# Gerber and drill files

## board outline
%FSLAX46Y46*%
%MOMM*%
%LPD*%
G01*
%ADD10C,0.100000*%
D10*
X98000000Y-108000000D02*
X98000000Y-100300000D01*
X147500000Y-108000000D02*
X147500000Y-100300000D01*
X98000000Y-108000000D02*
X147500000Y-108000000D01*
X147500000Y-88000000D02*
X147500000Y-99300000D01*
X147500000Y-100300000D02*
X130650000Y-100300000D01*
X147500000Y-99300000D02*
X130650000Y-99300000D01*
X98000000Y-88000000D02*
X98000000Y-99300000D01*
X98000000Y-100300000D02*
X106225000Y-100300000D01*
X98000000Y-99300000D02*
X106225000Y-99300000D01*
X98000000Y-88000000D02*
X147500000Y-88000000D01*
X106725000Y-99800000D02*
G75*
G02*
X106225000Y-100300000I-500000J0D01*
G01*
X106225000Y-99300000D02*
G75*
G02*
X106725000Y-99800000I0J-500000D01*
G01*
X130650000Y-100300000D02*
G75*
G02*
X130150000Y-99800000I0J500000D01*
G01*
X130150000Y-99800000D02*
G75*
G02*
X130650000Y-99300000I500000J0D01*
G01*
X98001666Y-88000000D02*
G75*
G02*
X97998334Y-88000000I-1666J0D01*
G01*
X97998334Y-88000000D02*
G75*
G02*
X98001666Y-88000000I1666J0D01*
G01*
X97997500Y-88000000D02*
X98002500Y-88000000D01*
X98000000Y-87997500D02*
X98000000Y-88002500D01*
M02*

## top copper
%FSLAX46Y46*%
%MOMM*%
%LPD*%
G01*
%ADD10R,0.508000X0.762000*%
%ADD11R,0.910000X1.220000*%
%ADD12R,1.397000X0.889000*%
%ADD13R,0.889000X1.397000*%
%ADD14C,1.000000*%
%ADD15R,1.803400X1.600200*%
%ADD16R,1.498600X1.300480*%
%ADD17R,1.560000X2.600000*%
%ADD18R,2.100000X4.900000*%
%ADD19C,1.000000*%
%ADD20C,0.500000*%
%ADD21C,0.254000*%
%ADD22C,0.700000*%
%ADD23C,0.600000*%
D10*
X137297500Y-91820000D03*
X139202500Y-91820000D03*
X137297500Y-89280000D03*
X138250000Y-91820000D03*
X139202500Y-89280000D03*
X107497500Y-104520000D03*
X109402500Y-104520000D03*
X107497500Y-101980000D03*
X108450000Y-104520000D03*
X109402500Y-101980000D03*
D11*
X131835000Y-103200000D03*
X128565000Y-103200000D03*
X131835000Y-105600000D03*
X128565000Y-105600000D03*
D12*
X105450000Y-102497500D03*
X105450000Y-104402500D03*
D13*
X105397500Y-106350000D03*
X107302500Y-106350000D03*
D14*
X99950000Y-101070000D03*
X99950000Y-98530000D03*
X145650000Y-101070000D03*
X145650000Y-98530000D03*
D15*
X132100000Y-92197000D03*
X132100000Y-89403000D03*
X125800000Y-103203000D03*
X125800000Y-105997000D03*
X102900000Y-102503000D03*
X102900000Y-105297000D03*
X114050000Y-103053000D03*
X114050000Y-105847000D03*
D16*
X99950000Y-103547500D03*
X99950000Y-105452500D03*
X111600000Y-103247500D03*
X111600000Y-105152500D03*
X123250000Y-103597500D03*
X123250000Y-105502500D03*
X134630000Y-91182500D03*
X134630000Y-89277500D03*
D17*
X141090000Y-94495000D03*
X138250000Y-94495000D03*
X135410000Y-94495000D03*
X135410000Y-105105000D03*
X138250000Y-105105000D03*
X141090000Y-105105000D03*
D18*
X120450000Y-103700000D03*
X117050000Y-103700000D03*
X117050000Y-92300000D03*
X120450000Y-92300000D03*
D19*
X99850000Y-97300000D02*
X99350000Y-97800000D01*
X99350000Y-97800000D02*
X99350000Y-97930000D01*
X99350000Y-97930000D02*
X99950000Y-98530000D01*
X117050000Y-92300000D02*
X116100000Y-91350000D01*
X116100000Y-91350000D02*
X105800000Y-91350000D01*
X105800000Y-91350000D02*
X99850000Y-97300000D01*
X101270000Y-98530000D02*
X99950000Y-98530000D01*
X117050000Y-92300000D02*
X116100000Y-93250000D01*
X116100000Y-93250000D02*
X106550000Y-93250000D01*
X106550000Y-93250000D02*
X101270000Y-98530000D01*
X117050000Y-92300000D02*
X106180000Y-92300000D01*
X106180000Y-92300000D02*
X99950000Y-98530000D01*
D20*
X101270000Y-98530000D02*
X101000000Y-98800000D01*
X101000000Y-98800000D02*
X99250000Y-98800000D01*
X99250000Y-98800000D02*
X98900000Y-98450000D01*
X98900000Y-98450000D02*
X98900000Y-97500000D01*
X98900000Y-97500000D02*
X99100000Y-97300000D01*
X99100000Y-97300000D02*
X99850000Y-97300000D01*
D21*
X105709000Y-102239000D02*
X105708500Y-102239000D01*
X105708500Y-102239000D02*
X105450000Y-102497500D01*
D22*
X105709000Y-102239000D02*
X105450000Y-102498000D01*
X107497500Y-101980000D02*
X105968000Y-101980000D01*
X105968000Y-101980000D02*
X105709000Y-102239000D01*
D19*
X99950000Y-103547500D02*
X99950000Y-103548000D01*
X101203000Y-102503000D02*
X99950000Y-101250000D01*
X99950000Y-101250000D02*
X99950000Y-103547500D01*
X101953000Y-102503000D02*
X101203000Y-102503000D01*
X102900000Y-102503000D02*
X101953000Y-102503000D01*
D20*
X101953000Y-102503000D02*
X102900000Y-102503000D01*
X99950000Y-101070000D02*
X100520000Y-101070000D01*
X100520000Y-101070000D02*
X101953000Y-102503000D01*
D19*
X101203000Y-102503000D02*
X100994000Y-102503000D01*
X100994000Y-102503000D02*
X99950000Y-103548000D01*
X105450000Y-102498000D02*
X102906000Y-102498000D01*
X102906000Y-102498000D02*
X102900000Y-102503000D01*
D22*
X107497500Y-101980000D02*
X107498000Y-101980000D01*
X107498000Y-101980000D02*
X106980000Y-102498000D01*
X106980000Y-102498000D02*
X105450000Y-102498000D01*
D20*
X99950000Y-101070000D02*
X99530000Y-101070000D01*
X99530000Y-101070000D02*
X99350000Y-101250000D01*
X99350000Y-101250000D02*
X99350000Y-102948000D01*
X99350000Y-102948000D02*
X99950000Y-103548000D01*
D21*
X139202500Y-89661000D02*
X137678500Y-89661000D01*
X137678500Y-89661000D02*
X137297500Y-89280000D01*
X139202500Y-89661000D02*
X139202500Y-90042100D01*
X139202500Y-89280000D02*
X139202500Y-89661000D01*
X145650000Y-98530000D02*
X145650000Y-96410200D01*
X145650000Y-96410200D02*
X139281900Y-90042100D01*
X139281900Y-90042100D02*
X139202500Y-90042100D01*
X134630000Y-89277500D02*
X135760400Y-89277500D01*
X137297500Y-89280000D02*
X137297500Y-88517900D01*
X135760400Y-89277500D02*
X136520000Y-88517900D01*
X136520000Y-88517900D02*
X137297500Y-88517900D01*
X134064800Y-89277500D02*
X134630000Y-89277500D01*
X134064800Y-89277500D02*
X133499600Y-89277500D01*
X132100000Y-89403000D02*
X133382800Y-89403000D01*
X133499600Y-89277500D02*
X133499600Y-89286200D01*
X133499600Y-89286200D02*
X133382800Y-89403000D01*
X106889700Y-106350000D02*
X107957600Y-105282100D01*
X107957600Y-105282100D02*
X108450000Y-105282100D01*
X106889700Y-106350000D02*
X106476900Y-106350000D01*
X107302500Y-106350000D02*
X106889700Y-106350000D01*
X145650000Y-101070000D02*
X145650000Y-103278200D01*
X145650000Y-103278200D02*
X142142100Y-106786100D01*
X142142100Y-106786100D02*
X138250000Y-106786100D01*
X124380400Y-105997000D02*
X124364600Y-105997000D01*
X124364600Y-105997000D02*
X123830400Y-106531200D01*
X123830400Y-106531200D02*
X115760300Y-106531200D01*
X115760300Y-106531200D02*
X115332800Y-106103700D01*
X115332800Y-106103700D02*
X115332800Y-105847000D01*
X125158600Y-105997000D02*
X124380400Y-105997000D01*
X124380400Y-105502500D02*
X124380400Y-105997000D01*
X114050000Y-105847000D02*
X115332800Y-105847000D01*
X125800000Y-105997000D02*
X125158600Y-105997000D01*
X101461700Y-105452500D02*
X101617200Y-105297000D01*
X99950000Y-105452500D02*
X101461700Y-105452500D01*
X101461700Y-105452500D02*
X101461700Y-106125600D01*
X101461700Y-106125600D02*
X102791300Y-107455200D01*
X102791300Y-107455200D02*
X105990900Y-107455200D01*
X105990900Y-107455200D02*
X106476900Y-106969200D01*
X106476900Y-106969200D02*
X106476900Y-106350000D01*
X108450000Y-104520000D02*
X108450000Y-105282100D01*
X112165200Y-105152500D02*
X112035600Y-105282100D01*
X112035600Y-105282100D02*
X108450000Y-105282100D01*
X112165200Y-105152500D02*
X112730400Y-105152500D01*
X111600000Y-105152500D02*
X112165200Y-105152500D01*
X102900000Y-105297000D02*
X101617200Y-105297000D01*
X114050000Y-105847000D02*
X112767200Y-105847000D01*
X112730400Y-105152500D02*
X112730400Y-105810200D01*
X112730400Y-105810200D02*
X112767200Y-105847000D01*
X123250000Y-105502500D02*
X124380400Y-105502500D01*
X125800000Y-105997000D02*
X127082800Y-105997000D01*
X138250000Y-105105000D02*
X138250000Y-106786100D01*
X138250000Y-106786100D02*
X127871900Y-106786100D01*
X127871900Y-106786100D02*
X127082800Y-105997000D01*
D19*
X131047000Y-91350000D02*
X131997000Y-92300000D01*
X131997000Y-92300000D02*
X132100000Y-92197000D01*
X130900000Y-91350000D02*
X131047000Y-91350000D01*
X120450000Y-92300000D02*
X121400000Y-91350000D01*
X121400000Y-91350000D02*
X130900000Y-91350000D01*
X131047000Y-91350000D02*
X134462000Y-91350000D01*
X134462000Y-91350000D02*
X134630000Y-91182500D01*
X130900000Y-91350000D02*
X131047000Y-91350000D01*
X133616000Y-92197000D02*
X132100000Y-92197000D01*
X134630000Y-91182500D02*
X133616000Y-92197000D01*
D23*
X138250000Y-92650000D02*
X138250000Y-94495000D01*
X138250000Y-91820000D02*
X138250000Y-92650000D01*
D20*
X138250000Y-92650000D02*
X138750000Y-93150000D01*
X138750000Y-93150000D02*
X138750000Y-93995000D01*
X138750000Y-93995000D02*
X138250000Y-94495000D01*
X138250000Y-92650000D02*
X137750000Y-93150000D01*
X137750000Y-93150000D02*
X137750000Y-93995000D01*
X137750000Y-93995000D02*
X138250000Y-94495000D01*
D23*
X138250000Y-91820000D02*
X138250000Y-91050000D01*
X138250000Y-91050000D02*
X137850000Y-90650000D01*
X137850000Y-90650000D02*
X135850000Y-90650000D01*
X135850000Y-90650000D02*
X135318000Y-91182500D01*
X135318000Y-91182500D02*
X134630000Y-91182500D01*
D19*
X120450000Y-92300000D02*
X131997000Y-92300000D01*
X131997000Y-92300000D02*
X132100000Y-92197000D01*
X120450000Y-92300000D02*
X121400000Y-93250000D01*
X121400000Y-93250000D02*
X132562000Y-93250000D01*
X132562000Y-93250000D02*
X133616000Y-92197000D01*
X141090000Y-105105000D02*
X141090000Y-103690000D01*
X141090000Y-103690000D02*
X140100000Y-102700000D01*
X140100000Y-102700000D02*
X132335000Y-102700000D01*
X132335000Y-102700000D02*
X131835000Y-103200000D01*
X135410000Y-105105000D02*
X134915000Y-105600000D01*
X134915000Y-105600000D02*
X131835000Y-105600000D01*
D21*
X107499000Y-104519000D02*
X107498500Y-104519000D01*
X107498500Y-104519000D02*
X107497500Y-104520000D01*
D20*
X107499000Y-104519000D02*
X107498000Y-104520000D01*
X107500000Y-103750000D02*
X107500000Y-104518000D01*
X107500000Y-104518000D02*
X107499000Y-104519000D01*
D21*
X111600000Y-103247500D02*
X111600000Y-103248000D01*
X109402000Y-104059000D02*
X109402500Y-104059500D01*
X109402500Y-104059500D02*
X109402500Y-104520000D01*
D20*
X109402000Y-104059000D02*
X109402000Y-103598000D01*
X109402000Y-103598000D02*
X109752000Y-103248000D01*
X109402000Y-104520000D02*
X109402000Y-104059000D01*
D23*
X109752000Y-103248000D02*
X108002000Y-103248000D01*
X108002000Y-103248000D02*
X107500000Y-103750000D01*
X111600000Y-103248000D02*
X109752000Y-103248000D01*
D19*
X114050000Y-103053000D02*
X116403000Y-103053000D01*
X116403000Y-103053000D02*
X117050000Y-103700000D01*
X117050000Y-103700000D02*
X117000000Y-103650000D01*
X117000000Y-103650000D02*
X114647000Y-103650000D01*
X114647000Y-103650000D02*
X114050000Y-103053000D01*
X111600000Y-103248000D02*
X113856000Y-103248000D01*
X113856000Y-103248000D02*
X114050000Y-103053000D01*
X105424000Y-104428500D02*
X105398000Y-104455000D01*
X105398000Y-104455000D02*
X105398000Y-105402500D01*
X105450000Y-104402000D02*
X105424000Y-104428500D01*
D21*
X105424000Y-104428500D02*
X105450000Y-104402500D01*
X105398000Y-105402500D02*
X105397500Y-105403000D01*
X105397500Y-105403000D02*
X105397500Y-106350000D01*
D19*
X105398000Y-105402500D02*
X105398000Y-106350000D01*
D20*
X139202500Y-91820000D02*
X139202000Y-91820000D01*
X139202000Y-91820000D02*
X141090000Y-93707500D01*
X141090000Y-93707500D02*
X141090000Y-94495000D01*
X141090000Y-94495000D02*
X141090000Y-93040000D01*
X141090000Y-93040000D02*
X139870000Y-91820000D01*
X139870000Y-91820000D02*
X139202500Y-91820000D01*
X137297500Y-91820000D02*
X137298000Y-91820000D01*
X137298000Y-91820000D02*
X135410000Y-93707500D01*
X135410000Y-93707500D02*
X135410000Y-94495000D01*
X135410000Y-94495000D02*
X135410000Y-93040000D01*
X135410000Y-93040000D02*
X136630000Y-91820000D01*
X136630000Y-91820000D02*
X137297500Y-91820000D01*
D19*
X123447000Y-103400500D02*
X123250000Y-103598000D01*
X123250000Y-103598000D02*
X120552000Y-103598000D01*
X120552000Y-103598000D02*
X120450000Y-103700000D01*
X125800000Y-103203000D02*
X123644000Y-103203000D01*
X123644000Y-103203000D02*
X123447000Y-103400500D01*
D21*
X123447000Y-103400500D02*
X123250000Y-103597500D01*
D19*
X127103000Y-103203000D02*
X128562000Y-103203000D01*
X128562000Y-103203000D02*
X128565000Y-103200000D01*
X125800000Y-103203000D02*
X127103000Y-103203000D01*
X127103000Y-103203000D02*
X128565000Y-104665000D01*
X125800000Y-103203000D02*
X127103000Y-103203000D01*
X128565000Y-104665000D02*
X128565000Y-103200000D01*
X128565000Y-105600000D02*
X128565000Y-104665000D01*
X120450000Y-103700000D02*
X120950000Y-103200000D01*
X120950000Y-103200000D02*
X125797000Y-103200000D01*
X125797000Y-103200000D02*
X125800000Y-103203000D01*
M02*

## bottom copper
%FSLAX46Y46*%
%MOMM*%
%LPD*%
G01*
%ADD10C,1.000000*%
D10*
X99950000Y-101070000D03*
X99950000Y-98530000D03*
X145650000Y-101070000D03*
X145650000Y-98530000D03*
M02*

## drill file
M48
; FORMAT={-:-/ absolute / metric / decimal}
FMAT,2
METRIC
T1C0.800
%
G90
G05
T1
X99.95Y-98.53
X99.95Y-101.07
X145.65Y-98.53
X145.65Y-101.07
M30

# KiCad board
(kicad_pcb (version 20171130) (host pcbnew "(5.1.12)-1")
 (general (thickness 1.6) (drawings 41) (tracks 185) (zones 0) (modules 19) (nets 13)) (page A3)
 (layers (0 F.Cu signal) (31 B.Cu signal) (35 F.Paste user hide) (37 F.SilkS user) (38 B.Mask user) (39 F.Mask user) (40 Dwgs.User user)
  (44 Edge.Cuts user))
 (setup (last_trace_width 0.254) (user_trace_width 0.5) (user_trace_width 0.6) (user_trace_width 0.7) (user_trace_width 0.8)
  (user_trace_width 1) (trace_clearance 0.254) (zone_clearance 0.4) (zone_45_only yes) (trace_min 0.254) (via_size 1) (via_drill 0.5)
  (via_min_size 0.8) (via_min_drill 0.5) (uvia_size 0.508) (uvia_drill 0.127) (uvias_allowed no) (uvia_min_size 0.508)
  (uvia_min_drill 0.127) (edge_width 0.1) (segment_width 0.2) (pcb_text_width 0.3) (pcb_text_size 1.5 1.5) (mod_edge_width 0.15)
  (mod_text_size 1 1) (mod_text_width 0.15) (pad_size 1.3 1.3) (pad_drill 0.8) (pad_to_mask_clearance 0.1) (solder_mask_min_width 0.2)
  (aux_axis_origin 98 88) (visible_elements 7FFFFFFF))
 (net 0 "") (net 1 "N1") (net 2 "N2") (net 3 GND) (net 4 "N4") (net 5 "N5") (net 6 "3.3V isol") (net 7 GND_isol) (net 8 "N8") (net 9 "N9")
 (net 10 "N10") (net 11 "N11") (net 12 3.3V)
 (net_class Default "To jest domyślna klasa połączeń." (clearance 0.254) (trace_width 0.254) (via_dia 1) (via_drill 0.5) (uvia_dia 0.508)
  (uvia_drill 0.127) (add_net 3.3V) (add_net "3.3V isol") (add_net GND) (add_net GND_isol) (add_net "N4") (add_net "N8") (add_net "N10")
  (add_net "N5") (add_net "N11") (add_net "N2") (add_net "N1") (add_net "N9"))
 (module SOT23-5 (layer F.Cu) (at 138.25 90.55)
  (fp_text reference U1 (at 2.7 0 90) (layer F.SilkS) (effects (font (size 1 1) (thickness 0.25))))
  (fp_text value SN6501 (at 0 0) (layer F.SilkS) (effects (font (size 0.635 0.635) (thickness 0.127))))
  (pad 1 smd rect (at -0.9525 1.27) (size 0.508 0.762) (layers F.Cu F.Paste F.Mask) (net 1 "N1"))
  (pad 3 smd rect (at 0.9525 1.27) (size 0.508 0.762) (layers F.Cu F.Paste F.Mask) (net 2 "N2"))
  (pad 5 smd rect (at -0.9525 -1.27) (size 0.508 0.762) (layers F.Cu F.Paste F.Mask) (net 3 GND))
  (pad 2 smd rect (at 0 1.27) (size 0.508 0.762) (layers F.Cu F.Paste F.Mask) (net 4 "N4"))
  (pad 4 smd rect (at 0.9525 -1.27) (size 0.508 0.762) (layers F.Cu F.Paste F.Mask) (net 3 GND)))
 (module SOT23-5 (layer F.Cu) (at 108.45 103.25)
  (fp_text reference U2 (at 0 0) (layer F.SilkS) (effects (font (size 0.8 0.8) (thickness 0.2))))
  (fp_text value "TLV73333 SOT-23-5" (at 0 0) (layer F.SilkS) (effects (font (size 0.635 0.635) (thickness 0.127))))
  (pad 1 smd rect (at -0.9525 1.27) (size 0.508 0.762) (layers F.Cu F.Paste F.Mask) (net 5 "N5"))
  (pad 3 smd rect (at 0.9525 1.27) (size 0.508 0.762) (layers F.Cu F.Paste F.Mask) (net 5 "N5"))
  (pad 5 smd rect (at -0.9525 -1.27) (size 0.508 0.762) (layers F.Cu F.Paste F.Mask) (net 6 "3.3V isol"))
  (pad 2 smd rect (at 0 1.27) (size 0.508 0.762) (layers F.Cu F.Paste F.Mask) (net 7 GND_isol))
  (pad 4 smd rect (at 0.9525 -1.27) (size 0.508 0.762) (layers F.Cu F.Paste F.Mask)))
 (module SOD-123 (layer F.Cu) (at 130.2 103.2 180)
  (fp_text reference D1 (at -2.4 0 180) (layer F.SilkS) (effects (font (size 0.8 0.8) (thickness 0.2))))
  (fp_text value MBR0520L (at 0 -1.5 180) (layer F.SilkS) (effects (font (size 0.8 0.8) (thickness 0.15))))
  (pad 1 smd rect (at -1.635 0 180) (size 0.91 1.22) (layers F.Cu F.Paste F.Mask) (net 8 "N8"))
  (pad 2 smd rect (at 1.635 0 180) (size 0.91 1.22) (layers F.Cu F.Paste F.Mask) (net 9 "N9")))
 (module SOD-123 (layer F.Cu) (at 130.2 105.6 180)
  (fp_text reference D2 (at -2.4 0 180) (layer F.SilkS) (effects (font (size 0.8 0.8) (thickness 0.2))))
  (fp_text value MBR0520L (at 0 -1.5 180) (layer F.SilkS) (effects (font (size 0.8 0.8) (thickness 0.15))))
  (pad 1 smd rect (at -1.635 0 180) (size 0.91 1.22) (layers F.Cu F.Paste F.Mask) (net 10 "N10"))
  (pad 2 smd rect (at 1.635 0 180) (size 0.91 1.22) (layers F.Cu F.Paste F.Mask) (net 9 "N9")))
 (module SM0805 (layer F.Cu) (at 105.45 103.45 270)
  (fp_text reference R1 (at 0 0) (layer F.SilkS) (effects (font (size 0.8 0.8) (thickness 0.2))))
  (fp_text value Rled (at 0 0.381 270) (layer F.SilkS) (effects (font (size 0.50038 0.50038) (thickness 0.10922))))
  (pad 1 smd rect (at -0.9525 0 270) (size 0.889 1.397) (layers F.Cu F.Paste F.Mask) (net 6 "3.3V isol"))
  (pad 2 smd rect (at 0.9525 0 270) (size 0.889 1.397) (layers F.Cu F.Paste F.Mask) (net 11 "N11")))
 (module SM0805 (layer F.Cu) (at 106.35 106.35)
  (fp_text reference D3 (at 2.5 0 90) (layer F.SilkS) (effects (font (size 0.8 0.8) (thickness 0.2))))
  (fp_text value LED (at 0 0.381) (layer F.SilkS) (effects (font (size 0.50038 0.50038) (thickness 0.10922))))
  (pad 1 smd rect (at -0.9525 0) (size 0.889 1.397) (layers F.Cu F.Paste F.Mask) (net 11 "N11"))
  (pad 2 smd rect (at 0.9525 0) (size 0.889 1.397) (layers F.Cu F.Paste F.Mask) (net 7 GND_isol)))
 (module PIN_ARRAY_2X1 (layer F.Cu) (at 99.95 99.8 90)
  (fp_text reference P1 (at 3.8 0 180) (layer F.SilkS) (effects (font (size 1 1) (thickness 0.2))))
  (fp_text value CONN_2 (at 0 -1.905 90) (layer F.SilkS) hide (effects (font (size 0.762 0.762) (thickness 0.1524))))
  (pad 1 thru_hole circle (at -1.27 0 90) (size 1 1) (drill 0.8) (layers *.Cu *.Mask F.SilkS) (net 6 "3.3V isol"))
  (pad 2 thru_hole circle (at 1.27 0 90) (size 1 1) (drill 0.8) (layers *.Cu *.Mask F.SilkS) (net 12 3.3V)))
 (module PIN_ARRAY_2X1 (layer F.Cu) (at 145.65 99.8 90)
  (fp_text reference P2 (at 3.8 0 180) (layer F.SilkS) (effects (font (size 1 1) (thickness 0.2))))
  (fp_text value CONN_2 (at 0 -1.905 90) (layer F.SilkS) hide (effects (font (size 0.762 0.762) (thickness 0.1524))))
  (pad 1 thru_hole circle (at -1.27 0 90) (size 1 1) (drill 0.8) (layers *.Cu *.Mask F.SilkS) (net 7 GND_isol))
  (pad 2 thru_hole circle (at 1.27 0 90) (size 1 1) (drill 0.8) (layers *.Cu *.Mask F.SilkS) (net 3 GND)))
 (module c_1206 (layer F.Cu) (at 132.1 90.8 270)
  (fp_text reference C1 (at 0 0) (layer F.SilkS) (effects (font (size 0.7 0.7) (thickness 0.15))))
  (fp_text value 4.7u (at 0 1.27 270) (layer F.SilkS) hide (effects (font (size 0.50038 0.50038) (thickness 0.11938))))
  (pad 1 smd rect (at 1.397 0 270) (size 1.6002 1.8034) (layers F.Cu F.Paste F.Mask) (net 4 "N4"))
  (pad 2 smd rect (at -1.397 0 270) (size 1.6002 1.8034) (layers F.Cu F.Paste F.Mask) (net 3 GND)))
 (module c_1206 (layer F.Cu) (at 125.8 104.6 90)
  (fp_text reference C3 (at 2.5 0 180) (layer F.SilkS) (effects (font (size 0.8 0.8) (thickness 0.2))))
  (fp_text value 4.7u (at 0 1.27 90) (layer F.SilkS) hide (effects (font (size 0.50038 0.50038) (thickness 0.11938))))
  (pad 1 smd rect (at 1.397 0 90) (size 1.6002 1.8034) (layers F.Cu F.Paste F.Mask) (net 9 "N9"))
  (pad 2 smd rect (at -1.397 0 90) (size 1.6002 1.8034) (layers F.Cu F.Paste F.Mask) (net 7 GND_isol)))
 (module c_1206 (layer F.Cu) (at 102.9 103.9 90)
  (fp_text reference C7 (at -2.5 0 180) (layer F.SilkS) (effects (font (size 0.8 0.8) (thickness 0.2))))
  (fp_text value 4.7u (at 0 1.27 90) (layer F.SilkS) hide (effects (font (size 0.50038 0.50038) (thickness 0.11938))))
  (pad 1 smd rect (at 1.397 0 90) (size 1.6002 1.8034) (layers F.Cu F.Paste F.Mask) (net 6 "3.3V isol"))
  (pad 2 smd rect (at -1.397 0 90) (size 1.6002 1.8034) (layers F.Cu F.Paste F.Mask) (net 7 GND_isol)))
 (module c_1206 (layer F.Cu) (at 114.05 104.45 90)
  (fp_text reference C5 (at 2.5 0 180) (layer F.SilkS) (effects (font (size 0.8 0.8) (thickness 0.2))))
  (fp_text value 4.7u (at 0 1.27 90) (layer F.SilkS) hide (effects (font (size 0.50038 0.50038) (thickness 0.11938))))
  (pad 1 smd rect (at 1.397 0 90) (size 1.6002 1.8034) (layers F.Cu F.Paste F.Mask) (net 5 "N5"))
  (pad 2 smd rect (at -1.397 0 90) (size 1.6002 1.8034) (layers F.Cu F.Paste F.Mask) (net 7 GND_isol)))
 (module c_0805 (layer F.Cu) (at 99.95 104.5 90)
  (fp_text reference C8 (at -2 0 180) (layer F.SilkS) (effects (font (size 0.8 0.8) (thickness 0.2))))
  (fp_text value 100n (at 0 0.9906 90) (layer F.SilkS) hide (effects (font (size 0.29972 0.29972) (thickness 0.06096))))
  (pad 1 smd rect (at 0.9525 0 90) (size 1.30048 1.4986) (layers F.Cu F.Paste F.Mask) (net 6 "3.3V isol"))
  (pad 2 smd rect (at -0.9525 0 90) (size 1.30048 1.4986) (layers F.Cu F.Paste F.Mask) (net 7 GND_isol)))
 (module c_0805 (layer F.Cu) (at 111.6 104.2 90)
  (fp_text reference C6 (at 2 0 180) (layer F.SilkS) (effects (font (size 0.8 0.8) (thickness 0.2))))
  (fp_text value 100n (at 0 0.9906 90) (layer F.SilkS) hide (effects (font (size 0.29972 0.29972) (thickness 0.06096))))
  (pad 1 smd rect (at 0.9525 0 90) (size 1.30048 1.4986) (layers F.Cu F.Paste F.Mask) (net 5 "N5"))
  (pad 2 smd rect (at -0.9525 0 90) (size 1.30048 1.4986) (layers F.Cu F.Paste F.Mask) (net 7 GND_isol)))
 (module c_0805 (layer F.Cu) (at 123.25 104.55 90)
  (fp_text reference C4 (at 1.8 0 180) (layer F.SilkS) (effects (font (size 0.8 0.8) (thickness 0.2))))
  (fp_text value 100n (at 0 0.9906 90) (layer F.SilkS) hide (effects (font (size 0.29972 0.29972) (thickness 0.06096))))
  (pad 1 smd rect (at 0.9525 0 90) (size 1.30048 1.4986) (layers F.Cu F.Paste F.Mask) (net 9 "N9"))
  (pad 2 smd rect (at -0.9525 0 90) (size 1.30048 1.4986) (layers F.Cu F.Paste F.Mask) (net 7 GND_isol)))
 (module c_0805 (layer F.Cu) (at 134.63 90.23 270)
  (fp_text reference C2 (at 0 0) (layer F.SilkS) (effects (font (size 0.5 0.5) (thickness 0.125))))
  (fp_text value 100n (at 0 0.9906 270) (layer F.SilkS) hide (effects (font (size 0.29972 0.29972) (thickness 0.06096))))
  (pad 1 smd rect (at 0.9525 0 270) (size 1.30048 1.4986) (layers F.Cu F.Paste F.Mask) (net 4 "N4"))
  (pad 2 smd rect (at -0.9525 0 270) (size 1.30048 1.4986) (layers F.Cu F.Paste F.Mask) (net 3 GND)))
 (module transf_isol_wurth (layer F.Cu) (at 138.25 99.8 270)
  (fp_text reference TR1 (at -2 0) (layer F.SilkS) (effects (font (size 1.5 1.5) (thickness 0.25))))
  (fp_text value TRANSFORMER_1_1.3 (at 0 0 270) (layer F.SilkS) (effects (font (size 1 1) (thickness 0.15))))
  (pad 1 smd rect (at -5.305 -2.84 270) (size 2.6 1.56) (layers F.Cu F.Paste F.Mask) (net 2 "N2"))
  (pad 2 smd rect (at -5.305 0 270) (size 2.6 1.56) (layers F.Cu F.Paste F.Mask) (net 4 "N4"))
  (pad 3 smd rect (at -5.305 2.84 270) (size 2.6 1.56) (layers F.Cu F.Paste F.Mask) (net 1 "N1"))
  (pad 4 smd rect (at 5.305 2.84 270) (size 2.6 1.56) (layers F.Cu F.Paste F.Mask) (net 10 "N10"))
  (pad 5 smd rect (at 5.305 0 270) (size 2.6 1.56) (layers F.Cu F.Paste F.Mask) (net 7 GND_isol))
  (pad 6 smd rect (at 5.305 -2.84 270) (size 2.6 1.56) (layers F.Cu F.Paste F.Mask) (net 8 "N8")))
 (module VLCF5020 (layer F.Cu) (at 118.75 103.7 180)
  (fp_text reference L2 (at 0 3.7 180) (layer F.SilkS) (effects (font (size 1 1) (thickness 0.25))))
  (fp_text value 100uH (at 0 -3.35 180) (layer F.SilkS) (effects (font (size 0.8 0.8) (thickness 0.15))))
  (pad 1 smd rect (at -1.7 0 180) (size 2.1 4.9) (layers F.Cu F.Paste F.Mask) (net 9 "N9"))
  (pad 2 smd rect (at 1.7 0 180) (size 2.1 4.9) (layers F.Cu F.Paste F.Mask) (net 5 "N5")))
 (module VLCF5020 (layer F.Cu) (at 118.75 92.3)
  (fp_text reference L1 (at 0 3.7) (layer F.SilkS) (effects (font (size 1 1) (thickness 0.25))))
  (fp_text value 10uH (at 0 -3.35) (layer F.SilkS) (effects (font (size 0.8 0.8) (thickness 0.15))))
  (pad 1 smd rect (at -1.7 0) (size 2.1 4.9) (layers F.Cu F.Paste F.Mask) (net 12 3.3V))
  (pad 2 smd rect (at 1.7 0) (size 2.1 4.9) (layers F.Cu F.Paste F.Mask) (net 4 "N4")))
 (gr_line (start 98 108) (end 98 100.3) (angle 90) (layer Edge.Cuts) (width 0.1))
 (gr_line (start 147.5 108) (end 147.5 100.3) (angle 90) (layer Edge.Cuts) (width 0.1))
 (gr_line (start 98 108) (end 147.5 108) (angle 90) (layer Edge.Cuts) (width 0.1))
 (gr_line (start 147.5 88) (end 147.5 99.3) (angle 90) (layer Edge.Cuts) (width 0.1))
 (gr_line (start 147.5 100.3) (end 130.65 100.3) (angle 90) (layer Edge.Cuts) (width 0.1))
 (gr_line (start 147.5 99.3) (end 130.65 99.3) (angle 90) (layer Edge.Cuts) (width 0.1))
 (gr_line (start 98 88) (end 98 99.3) (angle 90) (layer Edge.Cuts) (width 0.1))
 (gr_line (start 98 100.3) (end 106.225 100.3) (angle 90) (layer Edge.Cuts) (width 0.1))
 (gr_line (start 98 99.3) (end 106.225 99.3) (angle 90) (layer Edge.Cuts) (width 0.1))
 (gr_line (start 98 88) (end 147.5 88) (angle 90) (layer Edge.Cuts) (width 0.1))
 (gr_arc (start 106.225 99.8) (end 106.725 99.8) (angle 90) (layer Edge.Cuts) (width 0.1))
 (gr_arc (start 106.225 99.8) (end 106.225 99.3) (angle 90) (layer Edge.Cuts) (width 0.1))
 (gr_arc (start 130.65 99.8) (end 130.65 100.3) (angle 90) (layer Edge.Cuts) (width 0.1))
 (gr_arc (start 130.65 99.8) (end 130.15 99.8) (angle 90) (layer Edge.Cuts) (width 0.1))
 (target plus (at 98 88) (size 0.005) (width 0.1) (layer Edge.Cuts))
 (segment (start 99.85 97.3) (end 99.35 97.8) (width 1) (layer F.Cu) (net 12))
 (segment (start 99.35 97.8) (end 99.35 97.93) (width 1) (layer F.Cu) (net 12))
 (segment (start 99.35 97.93) (end 99.95 98.53) (width 1) (layer F.Cu) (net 12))
 (segment (start 117.05 92.3) (end 116.1 91.35) (width 1) (layer F.Cu) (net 12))
 (segment (start 116.1 91.35) (end 105.8 91.35) (width 1) (layer F.Cu) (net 12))
 (segment (start 105.8 91.35) (end 99.85 97.3) (width 1) (layer F.Cu) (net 12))
 (segment (start 101.27 98.53) (end 99.95 98.53) (width 1) (layer F.Cu) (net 12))
 (segment (start 117.05 92.3) (end 116.1 93.25) (width 1) (layer F.Cu) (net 12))
 (segment (start 116.1 93.25) (end 106.55 93.25) (width 1) (layer F.Cu) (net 12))
 (segment (start 106.55 93.25) (end 101.27 98.53) (width 1) (layer F.Cu) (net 12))
 (segment (start 117.05 92.3) (end 106.18 92.3) (width 1) (layer F.Cu) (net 12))
 (segment (start 106.18 92.3) (end 99.95 98.53) (width 1) (layer F.Cu) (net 12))
 (segment (start 101.27 98.53) (end 101 98.8) (width 0.5) (layer F.Cu) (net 12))
 (segment (start 101 98.8) (end 99.25 98.8) (width 0.5) (layer F.Cu) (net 12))
 (segment (start 99.25 98.8) (end 98.9 98.45) (width 0.5) (layer F.Cu) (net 12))
 (segment (start 98.9 98.45) (end 98.9 97.5) (width 0.5) (layer F.Cu) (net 12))
 (segment (start 98.9 97.5) (end 99.1 97.3) (width 0.5) (layer F.Cu) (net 12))
 (segment (start 99.1 97.3) (end 99.85 97.3) (width 0.5) (layer F.Cu) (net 12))
 (segment (start 105.709 102.239) (end 105.7085 102.239) (width 0.254) (layer F.Cu) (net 6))
 (segment (start 105.7085 102.239) (end 105.45 102.4975) (width 0.254) (layer F.Cu) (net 6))
 (segment (start 105.709 102.239) (end 105.45 102.498) (width 0.7) (layer F.Cu) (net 6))
 (segment (start 107.4975 101.98) (end 105.968 101.98) (width 0.7) (layer F.Cu) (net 6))
 (segment (start 105.968 101.98) (end 105.709 102.239) (width 0.7) (layer F.Cu) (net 6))
 (segment (start 99.95 103.5475) (end 99.95 103.548) (width 1) (layer F.Cu) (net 6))
 (segment (start 101.203 102.503) (end 99.95 101.25) (width 1) (layer F.Cu) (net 6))
 (segment (start 99.95 101.25) (end 99.95 103.5475) (width 1) (layer F.Cu) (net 6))
 (segment (start 101.953 102.503) (end 101.203 102.503) (width 1) (layer F.Cu) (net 6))
 (segment (start 102.9 102.503) (end 101.953 102.503) (width 1) (layer F.Cu) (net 6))
 (segment (start 101.953 102.503) (end 102.9 102.503) (width 0.5) (layer F.Cu) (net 6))
 (segment (start 99.95 101.07) (end 100.52 101.07) (width 0.5) (layer F.Cu) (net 6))
 (segment (start 100.52 101.07) (end 101.953 102.503) (width 0.5) (layer F.Cu) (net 6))
 (segment (start 101.203 102.503) (end 100.994 102.503) (width 1) (layer F.Cu) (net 6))
 (segment (start 100.994 102.503) (end 99.95 103.548) (width 1) (layer F.Cu) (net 6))
 (segment (start 105.45 102.498) (end 102.906 102.498) (width 1) (layer F.Cu) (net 6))
 (segment (start 102.906 102.498) (end 102.9 102.503) (width 1) (layer F.Cu) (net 6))
 (segment (start 107.4975 101.98) (end 107.498 101.98) (width 0.7) (layer F.Cu) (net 6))
 (segment (start 107.498 101.98) (end 106.98 102.498) (width 0.7) (layer F.Cu) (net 6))
 (segment (start 106.98 102.498) (end 105.45 102.498) (width 0.7) (layer F.Cu) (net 6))
 (segment (start 99.95 101.07) (end 99.53 101.07) (width 0.5) (layer F.Cu) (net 6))
 (segment (start 99.53 101.07) (end 99.35 101.25) (width 0.5) (layer F.Cu) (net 6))
 (segment (start 99.35 101.25) (end 99.35 102.948) (width 0.5) (layer F.Cu) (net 6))
 (segment (start 99.35 102.948) (end 99.95 103.548) (width 0.5) (layer F.Cu) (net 6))
 (segment (start 139.2025 89.661) (end 137.6785 89.661) (width 0.254) (layer F.Cu) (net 3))
 (segment (start 137.6785 89.661) (end 137.2975 89.28) (width 0.254) (layer F.Cu) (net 3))
 (segment (start 139.2025 89.661) (end 139.2025 90.0421) (width 0.254) (layer F.Cu) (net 3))
 (segment (start 139.2025 89.28) (end 139.2025 89.661) (width 0.254) (layer F.Cu) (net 3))
 (segment (start 145.65 98.53) (end 145.65 96.4102) (width 0.254) (layer F.Cu) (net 3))
 (segment (start 145.65 96.4102) (end 139.2819 90.0421) (width 0.254) (layer F.Cu) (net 3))
 (segment (start 139.2819 90.0421) (end 139.2025 90.0421) (width 0.254) (layer F.Cu) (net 3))
 (segment (start 134.63 89.2775) (end 135.7604 89.2775) (width 0.254) (layer F.Cu) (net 3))
 (segment (start 137.2975 89.28) (end 137.2975 88.5179) (width 0.254) (layer F.Cu) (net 3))
 (segment (start 135.7604 89.2775) (end 136.52 88.5179) (width 0.254) (layer F.Cu) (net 3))
 (segment (start 136.52 88.5179) (end 137.2975 88.5179) (width 0.254) (layer F.Cu) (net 3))
 (segment (start 134.0648 89.2775) (end 134.63 89.2775) (width 0.254) (layer F.Cu) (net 3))
 (segment (start 134.0648 89.2775) (end 133.4996 89.2775) (width 0.254) (layer F.Cu) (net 3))
 (segment (start 132.1 89.403) (end 133.3828 89.403) (width 0.254) (layer F.Cu) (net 3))
 (segment (start 133.4996 89.2775) (end 133.4996 89.2862) (width 0.254) (layer F.Cu) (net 3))
 (segment (start 133.4996 89.2862) (end 133.3828 89.403) (width 0.254) (layer F.Cu) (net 3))
 (segment (start 106.8897 106.35) (end 107.9576 105.2821) (width 0.254) (layer F.Cu) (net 7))
 (segment (start 107.9576 105.2821) (end 108.45 105.2821) (width 0.254) (layer F.Cu) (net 7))
 (segment (start 106.8897 106.35) (end 106.4769 106.35) (width 0.254) (layer F.Cu) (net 7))
 (segment (start 107.3025 106.35) (end 106.8897 106.35) (width 0.254) (layer F.Cu) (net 7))
 (segment (start 145.65 101.07) (end 145.65 103.2782) (width 0.254) (layer F.Cu) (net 7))
 (segment (start 145.65 103.2782) (end 142.1421 106.7861) (width 0.254) (layer F.Cu) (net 7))
 (segment (start 142.1421 106.7861) (end 138.25 106.7861) (width 0.254) (layer F.Cu) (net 7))
 (segment (start 124.3804 105.997) (end 124.3646 105.997) (width 0.254) (layer F.Cu) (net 7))
 (segment (start 124.3646 105.997) (end 123.8304 106.5312) (width 0.254) (layer F.Cu) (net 7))
 (segment (start 123.8304 106.5312) (end 115.7603 106.5312) (width 0.254) (layer F.Cu) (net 7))
 (segment (start 115.7603 106.5312) (end 115.3328 106.1037) (width 0.254) (layer F.Cu) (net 7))
 (segment (start 115.3328 106.1037) (end 115.3328 105.847) (width 0.254) (layer F.Cu) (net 7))
 (segment (start 125.1586 105.997) (end 124.3804 105.997) (width 0.254) (layer F.Cu) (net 7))
 (segment (start 124.3804 105.5025) (end 124.3804 105.997) (width 0.254) (layer F.Cu) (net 7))
 (segment (start 114.05 105.847) (end 115.3328 105.847) (width 0.254) (layer F.Cu) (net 7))
 (segment (start 125.8 105.997) (end 125.1586 105.997) (width 0.254) (layer F.Cu) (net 7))
 (segment (start 101.4617 105.4525) (end 101.6172 105.297) (width 0.254) (layer F.Cu) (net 7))
 (segment (start 99.95 105.4525) (end 101.4617 105.4525) (width 0.254) (layer F.Cu) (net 7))
 (segment (start 101.4617 105.4525) (end 101.4617 106.1256) (width 0.254) (layer F.Cu) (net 7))
 (segment (start 101.4617 106.1256) (end 102.7913 107.4552) (width 0.254) (layer F.Cu) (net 7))
 (segment (start 102.7913 107.4552) (end 105.9909 107.4552) (width 0.254) (layer F.Cu) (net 7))
 (segment (start 105.9909 107.4552) (end 106.4769 106.9692) (width 0.254) (layer F.Cu) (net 7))
 (segment (start 106.4769 106.9692) (end 106.4769 106.35) (width 0.254) (layer F.Cu) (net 7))
 (segment (start 108.45 104.52) (end 108.45 105.2821) (width 0.254) (layer F.Cu) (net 7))
 (segment (start 112.1652 105.1525) (end 112.0356 105.2821) (width 0.254) (layer F.Cu) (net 7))
 (segment (start 112.0356 105.2821) (end 108.45 105.2821) (width 0.254) (layer F.Cu) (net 7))
 (segment (start 112.1652 105.1525) (end 112.7304 105.1525) (width 0.254) (layer F.Cu) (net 7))
 (segment (start 111.6 105.1525) (end 112.1652 105.1525) (width 0.254) (layer F.Cu) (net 7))
 (segment (start 102.9 105.297) (end 101.6172 105.297) (width 0.254) (layer F.Cu) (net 7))
 (segment (start 114.05 105.847) (end 112.7672 105.847) (width 0.254) (layer F.Cu) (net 7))
 (segment (start 112.7304 105.1525) (end 112.7304 105.8102) (width 0.254) (layer F.Cu) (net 7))
 (segment (start 112.7304 105.8102) (end 112.7672 105.847) (width 0.254) (layer F.Cu) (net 7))
 (segment (start 123.25 105.5025) (end 124.3804 105.5025) (width 0.254) (layer F.Cu) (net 7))
 (segment (start 125.8 105.997) (end 127.0828 105.997) (width 0.254) (layer F.Cu) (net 7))
 (segment (start 138.25 105.105) (end 138.25 106.7861) (width 0.254) (layer F.Cu) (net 7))
 (segment (start 138.25 106.7861) (end 127.8719 106.7861) (width 0.254) (layer F.Cu) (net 7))
 (segment (start 127.8719 106.7861) (end 127.0828 105.997) (width 0.254) (layer F.Cu) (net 7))
 (segment (start 131.047 91.35) (end 131.997 92.3) (width 1) (layer F.Cu) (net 4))
 (segment (start 131.997 92.3) (end 132.1 92.197) (width 1) (layer F.Cu) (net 4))
 (segment (start 130.9 91.35) (end 131.047 91.35) (width 1) (layer F.Cu) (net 4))
 (segment (start 120.45 92.3) (end 121.4 91.35) (width 1) (layer F.Cu) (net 4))
 (segment (start 121.4 91.35) (end 130.9 91.35) (width 1) (layer F.Cu) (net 4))
 (segment (start 131.047 91.35) (end 134.462 91.35) (width 1) (layer F.Cu) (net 4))
 (segment (start 134.462 91.35) (end 134.63 91.1825) (width 1) (layer F.Cu) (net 4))
 (segment (start 130.9 91.35) (end 131.047 91.35) (width 1) (layer F.Cu) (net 4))
 (segment (start 133.616 92.197) (end 132.1 92.197) (width 1) (layer F.Cu) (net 4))
 (segment (start 134.63 91.1825) (end 133.616 92.197) (width 1) (layer F.Cu) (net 4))
 (segment (start 138.25 92.65) (end 138.25 94.495) (width 0.6) (layer F.Cu) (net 4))
 (segment (start 138.25 91.82) (end 138.25 92.65) (width 0.6) (layer F.Cu) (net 4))
 (segment (start 138.25 92.65) (end 138.75 93.15) (width 0.5) (layer F.Cu) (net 4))
 (segment (start 138.75 93.15) (end 138.75 93.995) (width 0.5) (layer F.Cu) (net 4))
 (segment (start 138.75 93.995) (end 138.25 94.495) (width 0.5) (layer F.Cu) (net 4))
 (segment (start 138.25 92.65) (end 137.75 93.15) (width 0.5) (layer F.Cu) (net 4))
 (segment (start 137.75 93.15) (end 137.75 93.995) (width 0.5) (layer F.Cu) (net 4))
 (segment (start 137.75 93.995) (end 138.25 94.495) (width 0.5) (layer F.Cu) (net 4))
 (segment (start 138.25 91.82) (end 138.25 91.05) (width 0.6) (layer F.Cu) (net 4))
 (segment (start 138.25 91.05) (end 137.85 90.65) (width 0.6) (layer F.Cu) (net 4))
 (segment (start 137.85 90.65) (end 135.85 90.65) (width 0.6) (layer F.Cu) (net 4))
 (segment (start 135.85 90.65) (end 135.318 91.1825) (width 0.6) (layer F.Cu) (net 4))
 (segment (start 135.318 91.1825) (end 134.63 91.1825) (width 0.6) (layer F.Cu) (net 4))
 (segment (start 120.45 92.3) (end 131.997 92.3) (width 1) (layer F.Cu) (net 4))
 (segment (start 131.997 92.3) (end 132.1 92.197) (width 1) (layer F.Cu) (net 4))
 (segment (start 120.45 92.3) (end 121.4 93.25) (width 1) (layer F.Cu) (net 4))
 (segment (start 121.4 93.25) (end 132.562 93.25) (width 1) (layer F.Cu) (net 4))
 (segment (start 132.562 93.25) (end 133.616 92.197) (width 1) (layer F.Cu) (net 4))
 (segment (start 141.09 105.105) (end 141.09 103.69) (width 1) (layer F.Cu) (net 8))
 (segment (start 141.09 103.69) (end 140.1 102.7) (width 1) (layer F.Cu) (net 8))
 (segment (start 140.1 102.7) (end 132.335 102.7) (width 1) (layer F.Cu) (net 8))
 (segment (start 132.335 102.7) (end 131.835 103.2) (width 1) (layer F.Cu) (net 8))
 (segment (start 135.41 105.105) (end 134.915 105.6) (width 1) (layer F.Cu) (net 10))
 (segment (start 134.915 105.6) (end 131.835 105.6) (width 1) (layer F.Cu) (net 10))
 (segment (start 107.499 104.519) (end 107.4985 104.519) (width 0.254) (layer F.Cu) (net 5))
 (segment (start 107.4985 104.519) (end 107.4975 104.52) (width 0.254) (layer F.Cu) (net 5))
 (segment (start 107.499 104.519) (end 107.498 104.52) (width 0.5) (layer F.Cu) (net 5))
 (segment (start 107.5 103.75) (end 107.5 104.518) (width 0.5) (layer F.Cu) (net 5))
 (segment (start 107.5 104.518) (end 107.499 104.519) (width 0.5) (layer F.Cu) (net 5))
 (segment (start 111.6 103.2475) (end 111.6 103.248) (width 0.254) (layer F.Cu) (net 5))
 (segment (start 109.402 104.059) (end 109.4025 104.0595) (width 0.254) (layer F.Cu) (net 5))
 (segment (start 109.4025 104.0595) (end 109.4025 104.52) (width 0.254) (layer F.Cu) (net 5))
 (segment (start 109.402 104.059) (end 109.402 103.598) (width 0.5) (layer F.Cu) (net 5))
 (segment (start 109.402 103.598) (end 109.752 103.248) (width 0.5) (layer F.Cu) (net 5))
 (segment (start 109.402 104.52) (end 109.402 104.059) (width 0.5) (layer F.Cu) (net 5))
 (segment (start 109.752 103.248) (end 108.002 103.248) (width 0.6) (layer F.Cu) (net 5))
 (segment (start 108.002 103.248) (end 107.5 103.75) (width 0.6) (layer F.Cu) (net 5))
 (segment (start 111.6 103.248) (end 109.752 103.248) (width 0.6) (layer F.Cu) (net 5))
 (segment (start 114.05 103.053) (end 116.403 103.053) (width 1) (layer F.Cu) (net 5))
 (segment (start 116.403 103.053) (end 117.05 103.7) (width 1) (layer F.Cu) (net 5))
 (segment (start 117.05 103.7) (end 117 103.65) (width 1) (layer F.Cu) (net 5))
 (segment (start 117 103.65) (end 114.647 103.65) (width 1) (layer F.Cu) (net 5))
 (segment (start 114.647 103.65) (end 114.05 103.053) (width 1) (layer F.Cu) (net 5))
 (segment (start 111.6 103.248) (end 113.856 103.248) (width 1) (layer F.Cu) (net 5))
 (segment (start 113.856 103.248) (end 114.05 103.053) (width 1) (layer F.Cu) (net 5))
 (segment (start 105.424 104.4285) (end 105.398 104.455) (width 1) (layer F.Cu) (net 11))
 (segment (start 105.398 104.455) (end 105.398 105.4025) (width 1) (layer F.Cu) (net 11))
 (segment (start 105.45 104.402) (end 105.424 104.4285) (width 1) (layer F.Cu) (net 11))
 (segment (start 105.424 104.4285) (end 105.45 104.4025) (width 0.254) (layer F.Cu) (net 11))
 (segment (start 105.398 105.4025) (end 105.3975 105.403) (width 0.254) (layer F.Cu) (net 11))
 (segment (start 105.3975 105.403) (end 105.3975 106.35) (width 0.254) (layer F.Cu) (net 11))
 (segment (start 105.398 105.4025) (end 105.398 106.35) (width 1) (layer F.Cu) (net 11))
 (segment (start 139.2025 91.82) (end 139.202 91.82) (width 0.5) (layer F.Cu) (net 2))
 (segment (start 139.202 91.82) (end 141.09 93.7075) (width 0.5) (layer F.Cu) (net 2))
 (segment (start 141.09 93.7075) (end 141.09 94.495) (width 0.5) (layer F.Cu) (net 2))
 (segment (start 141.09 94.495) (end 141.09 93.04) (width 0.5) (layer F.Cu) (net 2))
 (segment (start 141.09 93.04) (end 139.87 91.82) (width 0.5) (layer F.Cu) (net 2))
 (segment (start 139.87 91.82) (end 139.2025 91.82) (width 0.5) (layer F.Cu) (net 2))
 (segment (start 137.2975 91.82) (end 137.298 91.82) (width 0.5) (layer F.Cu) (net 1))
 (segment (start 137.298 91.82) (end 135.41 93.7075) (width 0.5) (layer F.Cu) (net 1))
 (segment (start 135.41 93.7075) (end 135.41 94.495) (width 0.5) (layer F.Cu) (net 1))
 (segment (start 135.41 94.495) (end 135.41 93.04) (width 0.5) (layer F.Cu) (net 1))
 (segment (start 135.41 93.04) (end 136.63 91.82) (width 0.5) (layer F.Cu) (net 1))
 (segment (start 136.63 91.82) (end 137.2975 91.82) (width 0.5) (layer F.Cu) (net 1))
 (segment (start 123.447 103.4005) (end 123.25 103.598) (width 1) (layer F.Cu) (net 9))
 (segment (start 123.25 103.598) (end 120.552 103.598) (width 1) (layer F.Cu) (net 9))
 (segment (start 120.552 103.598) (end 120.45 103.7) (width 1) (layer F.Cu) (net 9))
 (segment (start 125.8 103.203) (end 123.644 103.203) (width 1) (layer F.Cu) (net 9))
 (segment (start 123.644 103.203) (end 123.447 103.4005) (width 1) (layer F.Cu) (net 9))
 (segment (start 123.447 103.4005) (end 123.25 103.5975) (width 0.254) (layer F.Cu) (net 9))
 (segment (start 127.103 103.203) (end 128.562 103.203) (width 1) (layer F.Cu) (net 9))
 (segment (start 128.562 103.203) (end 128.565 103.2) (width 1) (layer F.Cu) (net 9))
 (segment (start 125.8 103.203) (end 127.103 103.203) (width 1) (layer F.Cu) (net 9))
 (segment (start 127.103 103.203) (end 128.565 104.665) (width 1) (layer F.Cu) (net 9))
 (segment (start 125.8 103.203) (end 127.103 103.203) (width 1) (layer F.Cu) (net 9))
 (segment (start 128.565 104.665) (end 128.565 103.2) (width 1) (layer F.Cu) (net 9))
 (segment (start 128.565 105.6) (end 128.565 104.665) (width 1) (layer F.Cu) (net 9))
 (segment (start 120.45 103.7) (end 120.95 103.2) (width 1) (layer F.Cu) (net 9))
 (segment (start 120.95 103.2) (end 125.797 103.2) (width 1) (layer F.Cu) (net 9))
 (segment (start 125.797 103.2) (end 125.8 103.203) (width 1) (layer F.Cu) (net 9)))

